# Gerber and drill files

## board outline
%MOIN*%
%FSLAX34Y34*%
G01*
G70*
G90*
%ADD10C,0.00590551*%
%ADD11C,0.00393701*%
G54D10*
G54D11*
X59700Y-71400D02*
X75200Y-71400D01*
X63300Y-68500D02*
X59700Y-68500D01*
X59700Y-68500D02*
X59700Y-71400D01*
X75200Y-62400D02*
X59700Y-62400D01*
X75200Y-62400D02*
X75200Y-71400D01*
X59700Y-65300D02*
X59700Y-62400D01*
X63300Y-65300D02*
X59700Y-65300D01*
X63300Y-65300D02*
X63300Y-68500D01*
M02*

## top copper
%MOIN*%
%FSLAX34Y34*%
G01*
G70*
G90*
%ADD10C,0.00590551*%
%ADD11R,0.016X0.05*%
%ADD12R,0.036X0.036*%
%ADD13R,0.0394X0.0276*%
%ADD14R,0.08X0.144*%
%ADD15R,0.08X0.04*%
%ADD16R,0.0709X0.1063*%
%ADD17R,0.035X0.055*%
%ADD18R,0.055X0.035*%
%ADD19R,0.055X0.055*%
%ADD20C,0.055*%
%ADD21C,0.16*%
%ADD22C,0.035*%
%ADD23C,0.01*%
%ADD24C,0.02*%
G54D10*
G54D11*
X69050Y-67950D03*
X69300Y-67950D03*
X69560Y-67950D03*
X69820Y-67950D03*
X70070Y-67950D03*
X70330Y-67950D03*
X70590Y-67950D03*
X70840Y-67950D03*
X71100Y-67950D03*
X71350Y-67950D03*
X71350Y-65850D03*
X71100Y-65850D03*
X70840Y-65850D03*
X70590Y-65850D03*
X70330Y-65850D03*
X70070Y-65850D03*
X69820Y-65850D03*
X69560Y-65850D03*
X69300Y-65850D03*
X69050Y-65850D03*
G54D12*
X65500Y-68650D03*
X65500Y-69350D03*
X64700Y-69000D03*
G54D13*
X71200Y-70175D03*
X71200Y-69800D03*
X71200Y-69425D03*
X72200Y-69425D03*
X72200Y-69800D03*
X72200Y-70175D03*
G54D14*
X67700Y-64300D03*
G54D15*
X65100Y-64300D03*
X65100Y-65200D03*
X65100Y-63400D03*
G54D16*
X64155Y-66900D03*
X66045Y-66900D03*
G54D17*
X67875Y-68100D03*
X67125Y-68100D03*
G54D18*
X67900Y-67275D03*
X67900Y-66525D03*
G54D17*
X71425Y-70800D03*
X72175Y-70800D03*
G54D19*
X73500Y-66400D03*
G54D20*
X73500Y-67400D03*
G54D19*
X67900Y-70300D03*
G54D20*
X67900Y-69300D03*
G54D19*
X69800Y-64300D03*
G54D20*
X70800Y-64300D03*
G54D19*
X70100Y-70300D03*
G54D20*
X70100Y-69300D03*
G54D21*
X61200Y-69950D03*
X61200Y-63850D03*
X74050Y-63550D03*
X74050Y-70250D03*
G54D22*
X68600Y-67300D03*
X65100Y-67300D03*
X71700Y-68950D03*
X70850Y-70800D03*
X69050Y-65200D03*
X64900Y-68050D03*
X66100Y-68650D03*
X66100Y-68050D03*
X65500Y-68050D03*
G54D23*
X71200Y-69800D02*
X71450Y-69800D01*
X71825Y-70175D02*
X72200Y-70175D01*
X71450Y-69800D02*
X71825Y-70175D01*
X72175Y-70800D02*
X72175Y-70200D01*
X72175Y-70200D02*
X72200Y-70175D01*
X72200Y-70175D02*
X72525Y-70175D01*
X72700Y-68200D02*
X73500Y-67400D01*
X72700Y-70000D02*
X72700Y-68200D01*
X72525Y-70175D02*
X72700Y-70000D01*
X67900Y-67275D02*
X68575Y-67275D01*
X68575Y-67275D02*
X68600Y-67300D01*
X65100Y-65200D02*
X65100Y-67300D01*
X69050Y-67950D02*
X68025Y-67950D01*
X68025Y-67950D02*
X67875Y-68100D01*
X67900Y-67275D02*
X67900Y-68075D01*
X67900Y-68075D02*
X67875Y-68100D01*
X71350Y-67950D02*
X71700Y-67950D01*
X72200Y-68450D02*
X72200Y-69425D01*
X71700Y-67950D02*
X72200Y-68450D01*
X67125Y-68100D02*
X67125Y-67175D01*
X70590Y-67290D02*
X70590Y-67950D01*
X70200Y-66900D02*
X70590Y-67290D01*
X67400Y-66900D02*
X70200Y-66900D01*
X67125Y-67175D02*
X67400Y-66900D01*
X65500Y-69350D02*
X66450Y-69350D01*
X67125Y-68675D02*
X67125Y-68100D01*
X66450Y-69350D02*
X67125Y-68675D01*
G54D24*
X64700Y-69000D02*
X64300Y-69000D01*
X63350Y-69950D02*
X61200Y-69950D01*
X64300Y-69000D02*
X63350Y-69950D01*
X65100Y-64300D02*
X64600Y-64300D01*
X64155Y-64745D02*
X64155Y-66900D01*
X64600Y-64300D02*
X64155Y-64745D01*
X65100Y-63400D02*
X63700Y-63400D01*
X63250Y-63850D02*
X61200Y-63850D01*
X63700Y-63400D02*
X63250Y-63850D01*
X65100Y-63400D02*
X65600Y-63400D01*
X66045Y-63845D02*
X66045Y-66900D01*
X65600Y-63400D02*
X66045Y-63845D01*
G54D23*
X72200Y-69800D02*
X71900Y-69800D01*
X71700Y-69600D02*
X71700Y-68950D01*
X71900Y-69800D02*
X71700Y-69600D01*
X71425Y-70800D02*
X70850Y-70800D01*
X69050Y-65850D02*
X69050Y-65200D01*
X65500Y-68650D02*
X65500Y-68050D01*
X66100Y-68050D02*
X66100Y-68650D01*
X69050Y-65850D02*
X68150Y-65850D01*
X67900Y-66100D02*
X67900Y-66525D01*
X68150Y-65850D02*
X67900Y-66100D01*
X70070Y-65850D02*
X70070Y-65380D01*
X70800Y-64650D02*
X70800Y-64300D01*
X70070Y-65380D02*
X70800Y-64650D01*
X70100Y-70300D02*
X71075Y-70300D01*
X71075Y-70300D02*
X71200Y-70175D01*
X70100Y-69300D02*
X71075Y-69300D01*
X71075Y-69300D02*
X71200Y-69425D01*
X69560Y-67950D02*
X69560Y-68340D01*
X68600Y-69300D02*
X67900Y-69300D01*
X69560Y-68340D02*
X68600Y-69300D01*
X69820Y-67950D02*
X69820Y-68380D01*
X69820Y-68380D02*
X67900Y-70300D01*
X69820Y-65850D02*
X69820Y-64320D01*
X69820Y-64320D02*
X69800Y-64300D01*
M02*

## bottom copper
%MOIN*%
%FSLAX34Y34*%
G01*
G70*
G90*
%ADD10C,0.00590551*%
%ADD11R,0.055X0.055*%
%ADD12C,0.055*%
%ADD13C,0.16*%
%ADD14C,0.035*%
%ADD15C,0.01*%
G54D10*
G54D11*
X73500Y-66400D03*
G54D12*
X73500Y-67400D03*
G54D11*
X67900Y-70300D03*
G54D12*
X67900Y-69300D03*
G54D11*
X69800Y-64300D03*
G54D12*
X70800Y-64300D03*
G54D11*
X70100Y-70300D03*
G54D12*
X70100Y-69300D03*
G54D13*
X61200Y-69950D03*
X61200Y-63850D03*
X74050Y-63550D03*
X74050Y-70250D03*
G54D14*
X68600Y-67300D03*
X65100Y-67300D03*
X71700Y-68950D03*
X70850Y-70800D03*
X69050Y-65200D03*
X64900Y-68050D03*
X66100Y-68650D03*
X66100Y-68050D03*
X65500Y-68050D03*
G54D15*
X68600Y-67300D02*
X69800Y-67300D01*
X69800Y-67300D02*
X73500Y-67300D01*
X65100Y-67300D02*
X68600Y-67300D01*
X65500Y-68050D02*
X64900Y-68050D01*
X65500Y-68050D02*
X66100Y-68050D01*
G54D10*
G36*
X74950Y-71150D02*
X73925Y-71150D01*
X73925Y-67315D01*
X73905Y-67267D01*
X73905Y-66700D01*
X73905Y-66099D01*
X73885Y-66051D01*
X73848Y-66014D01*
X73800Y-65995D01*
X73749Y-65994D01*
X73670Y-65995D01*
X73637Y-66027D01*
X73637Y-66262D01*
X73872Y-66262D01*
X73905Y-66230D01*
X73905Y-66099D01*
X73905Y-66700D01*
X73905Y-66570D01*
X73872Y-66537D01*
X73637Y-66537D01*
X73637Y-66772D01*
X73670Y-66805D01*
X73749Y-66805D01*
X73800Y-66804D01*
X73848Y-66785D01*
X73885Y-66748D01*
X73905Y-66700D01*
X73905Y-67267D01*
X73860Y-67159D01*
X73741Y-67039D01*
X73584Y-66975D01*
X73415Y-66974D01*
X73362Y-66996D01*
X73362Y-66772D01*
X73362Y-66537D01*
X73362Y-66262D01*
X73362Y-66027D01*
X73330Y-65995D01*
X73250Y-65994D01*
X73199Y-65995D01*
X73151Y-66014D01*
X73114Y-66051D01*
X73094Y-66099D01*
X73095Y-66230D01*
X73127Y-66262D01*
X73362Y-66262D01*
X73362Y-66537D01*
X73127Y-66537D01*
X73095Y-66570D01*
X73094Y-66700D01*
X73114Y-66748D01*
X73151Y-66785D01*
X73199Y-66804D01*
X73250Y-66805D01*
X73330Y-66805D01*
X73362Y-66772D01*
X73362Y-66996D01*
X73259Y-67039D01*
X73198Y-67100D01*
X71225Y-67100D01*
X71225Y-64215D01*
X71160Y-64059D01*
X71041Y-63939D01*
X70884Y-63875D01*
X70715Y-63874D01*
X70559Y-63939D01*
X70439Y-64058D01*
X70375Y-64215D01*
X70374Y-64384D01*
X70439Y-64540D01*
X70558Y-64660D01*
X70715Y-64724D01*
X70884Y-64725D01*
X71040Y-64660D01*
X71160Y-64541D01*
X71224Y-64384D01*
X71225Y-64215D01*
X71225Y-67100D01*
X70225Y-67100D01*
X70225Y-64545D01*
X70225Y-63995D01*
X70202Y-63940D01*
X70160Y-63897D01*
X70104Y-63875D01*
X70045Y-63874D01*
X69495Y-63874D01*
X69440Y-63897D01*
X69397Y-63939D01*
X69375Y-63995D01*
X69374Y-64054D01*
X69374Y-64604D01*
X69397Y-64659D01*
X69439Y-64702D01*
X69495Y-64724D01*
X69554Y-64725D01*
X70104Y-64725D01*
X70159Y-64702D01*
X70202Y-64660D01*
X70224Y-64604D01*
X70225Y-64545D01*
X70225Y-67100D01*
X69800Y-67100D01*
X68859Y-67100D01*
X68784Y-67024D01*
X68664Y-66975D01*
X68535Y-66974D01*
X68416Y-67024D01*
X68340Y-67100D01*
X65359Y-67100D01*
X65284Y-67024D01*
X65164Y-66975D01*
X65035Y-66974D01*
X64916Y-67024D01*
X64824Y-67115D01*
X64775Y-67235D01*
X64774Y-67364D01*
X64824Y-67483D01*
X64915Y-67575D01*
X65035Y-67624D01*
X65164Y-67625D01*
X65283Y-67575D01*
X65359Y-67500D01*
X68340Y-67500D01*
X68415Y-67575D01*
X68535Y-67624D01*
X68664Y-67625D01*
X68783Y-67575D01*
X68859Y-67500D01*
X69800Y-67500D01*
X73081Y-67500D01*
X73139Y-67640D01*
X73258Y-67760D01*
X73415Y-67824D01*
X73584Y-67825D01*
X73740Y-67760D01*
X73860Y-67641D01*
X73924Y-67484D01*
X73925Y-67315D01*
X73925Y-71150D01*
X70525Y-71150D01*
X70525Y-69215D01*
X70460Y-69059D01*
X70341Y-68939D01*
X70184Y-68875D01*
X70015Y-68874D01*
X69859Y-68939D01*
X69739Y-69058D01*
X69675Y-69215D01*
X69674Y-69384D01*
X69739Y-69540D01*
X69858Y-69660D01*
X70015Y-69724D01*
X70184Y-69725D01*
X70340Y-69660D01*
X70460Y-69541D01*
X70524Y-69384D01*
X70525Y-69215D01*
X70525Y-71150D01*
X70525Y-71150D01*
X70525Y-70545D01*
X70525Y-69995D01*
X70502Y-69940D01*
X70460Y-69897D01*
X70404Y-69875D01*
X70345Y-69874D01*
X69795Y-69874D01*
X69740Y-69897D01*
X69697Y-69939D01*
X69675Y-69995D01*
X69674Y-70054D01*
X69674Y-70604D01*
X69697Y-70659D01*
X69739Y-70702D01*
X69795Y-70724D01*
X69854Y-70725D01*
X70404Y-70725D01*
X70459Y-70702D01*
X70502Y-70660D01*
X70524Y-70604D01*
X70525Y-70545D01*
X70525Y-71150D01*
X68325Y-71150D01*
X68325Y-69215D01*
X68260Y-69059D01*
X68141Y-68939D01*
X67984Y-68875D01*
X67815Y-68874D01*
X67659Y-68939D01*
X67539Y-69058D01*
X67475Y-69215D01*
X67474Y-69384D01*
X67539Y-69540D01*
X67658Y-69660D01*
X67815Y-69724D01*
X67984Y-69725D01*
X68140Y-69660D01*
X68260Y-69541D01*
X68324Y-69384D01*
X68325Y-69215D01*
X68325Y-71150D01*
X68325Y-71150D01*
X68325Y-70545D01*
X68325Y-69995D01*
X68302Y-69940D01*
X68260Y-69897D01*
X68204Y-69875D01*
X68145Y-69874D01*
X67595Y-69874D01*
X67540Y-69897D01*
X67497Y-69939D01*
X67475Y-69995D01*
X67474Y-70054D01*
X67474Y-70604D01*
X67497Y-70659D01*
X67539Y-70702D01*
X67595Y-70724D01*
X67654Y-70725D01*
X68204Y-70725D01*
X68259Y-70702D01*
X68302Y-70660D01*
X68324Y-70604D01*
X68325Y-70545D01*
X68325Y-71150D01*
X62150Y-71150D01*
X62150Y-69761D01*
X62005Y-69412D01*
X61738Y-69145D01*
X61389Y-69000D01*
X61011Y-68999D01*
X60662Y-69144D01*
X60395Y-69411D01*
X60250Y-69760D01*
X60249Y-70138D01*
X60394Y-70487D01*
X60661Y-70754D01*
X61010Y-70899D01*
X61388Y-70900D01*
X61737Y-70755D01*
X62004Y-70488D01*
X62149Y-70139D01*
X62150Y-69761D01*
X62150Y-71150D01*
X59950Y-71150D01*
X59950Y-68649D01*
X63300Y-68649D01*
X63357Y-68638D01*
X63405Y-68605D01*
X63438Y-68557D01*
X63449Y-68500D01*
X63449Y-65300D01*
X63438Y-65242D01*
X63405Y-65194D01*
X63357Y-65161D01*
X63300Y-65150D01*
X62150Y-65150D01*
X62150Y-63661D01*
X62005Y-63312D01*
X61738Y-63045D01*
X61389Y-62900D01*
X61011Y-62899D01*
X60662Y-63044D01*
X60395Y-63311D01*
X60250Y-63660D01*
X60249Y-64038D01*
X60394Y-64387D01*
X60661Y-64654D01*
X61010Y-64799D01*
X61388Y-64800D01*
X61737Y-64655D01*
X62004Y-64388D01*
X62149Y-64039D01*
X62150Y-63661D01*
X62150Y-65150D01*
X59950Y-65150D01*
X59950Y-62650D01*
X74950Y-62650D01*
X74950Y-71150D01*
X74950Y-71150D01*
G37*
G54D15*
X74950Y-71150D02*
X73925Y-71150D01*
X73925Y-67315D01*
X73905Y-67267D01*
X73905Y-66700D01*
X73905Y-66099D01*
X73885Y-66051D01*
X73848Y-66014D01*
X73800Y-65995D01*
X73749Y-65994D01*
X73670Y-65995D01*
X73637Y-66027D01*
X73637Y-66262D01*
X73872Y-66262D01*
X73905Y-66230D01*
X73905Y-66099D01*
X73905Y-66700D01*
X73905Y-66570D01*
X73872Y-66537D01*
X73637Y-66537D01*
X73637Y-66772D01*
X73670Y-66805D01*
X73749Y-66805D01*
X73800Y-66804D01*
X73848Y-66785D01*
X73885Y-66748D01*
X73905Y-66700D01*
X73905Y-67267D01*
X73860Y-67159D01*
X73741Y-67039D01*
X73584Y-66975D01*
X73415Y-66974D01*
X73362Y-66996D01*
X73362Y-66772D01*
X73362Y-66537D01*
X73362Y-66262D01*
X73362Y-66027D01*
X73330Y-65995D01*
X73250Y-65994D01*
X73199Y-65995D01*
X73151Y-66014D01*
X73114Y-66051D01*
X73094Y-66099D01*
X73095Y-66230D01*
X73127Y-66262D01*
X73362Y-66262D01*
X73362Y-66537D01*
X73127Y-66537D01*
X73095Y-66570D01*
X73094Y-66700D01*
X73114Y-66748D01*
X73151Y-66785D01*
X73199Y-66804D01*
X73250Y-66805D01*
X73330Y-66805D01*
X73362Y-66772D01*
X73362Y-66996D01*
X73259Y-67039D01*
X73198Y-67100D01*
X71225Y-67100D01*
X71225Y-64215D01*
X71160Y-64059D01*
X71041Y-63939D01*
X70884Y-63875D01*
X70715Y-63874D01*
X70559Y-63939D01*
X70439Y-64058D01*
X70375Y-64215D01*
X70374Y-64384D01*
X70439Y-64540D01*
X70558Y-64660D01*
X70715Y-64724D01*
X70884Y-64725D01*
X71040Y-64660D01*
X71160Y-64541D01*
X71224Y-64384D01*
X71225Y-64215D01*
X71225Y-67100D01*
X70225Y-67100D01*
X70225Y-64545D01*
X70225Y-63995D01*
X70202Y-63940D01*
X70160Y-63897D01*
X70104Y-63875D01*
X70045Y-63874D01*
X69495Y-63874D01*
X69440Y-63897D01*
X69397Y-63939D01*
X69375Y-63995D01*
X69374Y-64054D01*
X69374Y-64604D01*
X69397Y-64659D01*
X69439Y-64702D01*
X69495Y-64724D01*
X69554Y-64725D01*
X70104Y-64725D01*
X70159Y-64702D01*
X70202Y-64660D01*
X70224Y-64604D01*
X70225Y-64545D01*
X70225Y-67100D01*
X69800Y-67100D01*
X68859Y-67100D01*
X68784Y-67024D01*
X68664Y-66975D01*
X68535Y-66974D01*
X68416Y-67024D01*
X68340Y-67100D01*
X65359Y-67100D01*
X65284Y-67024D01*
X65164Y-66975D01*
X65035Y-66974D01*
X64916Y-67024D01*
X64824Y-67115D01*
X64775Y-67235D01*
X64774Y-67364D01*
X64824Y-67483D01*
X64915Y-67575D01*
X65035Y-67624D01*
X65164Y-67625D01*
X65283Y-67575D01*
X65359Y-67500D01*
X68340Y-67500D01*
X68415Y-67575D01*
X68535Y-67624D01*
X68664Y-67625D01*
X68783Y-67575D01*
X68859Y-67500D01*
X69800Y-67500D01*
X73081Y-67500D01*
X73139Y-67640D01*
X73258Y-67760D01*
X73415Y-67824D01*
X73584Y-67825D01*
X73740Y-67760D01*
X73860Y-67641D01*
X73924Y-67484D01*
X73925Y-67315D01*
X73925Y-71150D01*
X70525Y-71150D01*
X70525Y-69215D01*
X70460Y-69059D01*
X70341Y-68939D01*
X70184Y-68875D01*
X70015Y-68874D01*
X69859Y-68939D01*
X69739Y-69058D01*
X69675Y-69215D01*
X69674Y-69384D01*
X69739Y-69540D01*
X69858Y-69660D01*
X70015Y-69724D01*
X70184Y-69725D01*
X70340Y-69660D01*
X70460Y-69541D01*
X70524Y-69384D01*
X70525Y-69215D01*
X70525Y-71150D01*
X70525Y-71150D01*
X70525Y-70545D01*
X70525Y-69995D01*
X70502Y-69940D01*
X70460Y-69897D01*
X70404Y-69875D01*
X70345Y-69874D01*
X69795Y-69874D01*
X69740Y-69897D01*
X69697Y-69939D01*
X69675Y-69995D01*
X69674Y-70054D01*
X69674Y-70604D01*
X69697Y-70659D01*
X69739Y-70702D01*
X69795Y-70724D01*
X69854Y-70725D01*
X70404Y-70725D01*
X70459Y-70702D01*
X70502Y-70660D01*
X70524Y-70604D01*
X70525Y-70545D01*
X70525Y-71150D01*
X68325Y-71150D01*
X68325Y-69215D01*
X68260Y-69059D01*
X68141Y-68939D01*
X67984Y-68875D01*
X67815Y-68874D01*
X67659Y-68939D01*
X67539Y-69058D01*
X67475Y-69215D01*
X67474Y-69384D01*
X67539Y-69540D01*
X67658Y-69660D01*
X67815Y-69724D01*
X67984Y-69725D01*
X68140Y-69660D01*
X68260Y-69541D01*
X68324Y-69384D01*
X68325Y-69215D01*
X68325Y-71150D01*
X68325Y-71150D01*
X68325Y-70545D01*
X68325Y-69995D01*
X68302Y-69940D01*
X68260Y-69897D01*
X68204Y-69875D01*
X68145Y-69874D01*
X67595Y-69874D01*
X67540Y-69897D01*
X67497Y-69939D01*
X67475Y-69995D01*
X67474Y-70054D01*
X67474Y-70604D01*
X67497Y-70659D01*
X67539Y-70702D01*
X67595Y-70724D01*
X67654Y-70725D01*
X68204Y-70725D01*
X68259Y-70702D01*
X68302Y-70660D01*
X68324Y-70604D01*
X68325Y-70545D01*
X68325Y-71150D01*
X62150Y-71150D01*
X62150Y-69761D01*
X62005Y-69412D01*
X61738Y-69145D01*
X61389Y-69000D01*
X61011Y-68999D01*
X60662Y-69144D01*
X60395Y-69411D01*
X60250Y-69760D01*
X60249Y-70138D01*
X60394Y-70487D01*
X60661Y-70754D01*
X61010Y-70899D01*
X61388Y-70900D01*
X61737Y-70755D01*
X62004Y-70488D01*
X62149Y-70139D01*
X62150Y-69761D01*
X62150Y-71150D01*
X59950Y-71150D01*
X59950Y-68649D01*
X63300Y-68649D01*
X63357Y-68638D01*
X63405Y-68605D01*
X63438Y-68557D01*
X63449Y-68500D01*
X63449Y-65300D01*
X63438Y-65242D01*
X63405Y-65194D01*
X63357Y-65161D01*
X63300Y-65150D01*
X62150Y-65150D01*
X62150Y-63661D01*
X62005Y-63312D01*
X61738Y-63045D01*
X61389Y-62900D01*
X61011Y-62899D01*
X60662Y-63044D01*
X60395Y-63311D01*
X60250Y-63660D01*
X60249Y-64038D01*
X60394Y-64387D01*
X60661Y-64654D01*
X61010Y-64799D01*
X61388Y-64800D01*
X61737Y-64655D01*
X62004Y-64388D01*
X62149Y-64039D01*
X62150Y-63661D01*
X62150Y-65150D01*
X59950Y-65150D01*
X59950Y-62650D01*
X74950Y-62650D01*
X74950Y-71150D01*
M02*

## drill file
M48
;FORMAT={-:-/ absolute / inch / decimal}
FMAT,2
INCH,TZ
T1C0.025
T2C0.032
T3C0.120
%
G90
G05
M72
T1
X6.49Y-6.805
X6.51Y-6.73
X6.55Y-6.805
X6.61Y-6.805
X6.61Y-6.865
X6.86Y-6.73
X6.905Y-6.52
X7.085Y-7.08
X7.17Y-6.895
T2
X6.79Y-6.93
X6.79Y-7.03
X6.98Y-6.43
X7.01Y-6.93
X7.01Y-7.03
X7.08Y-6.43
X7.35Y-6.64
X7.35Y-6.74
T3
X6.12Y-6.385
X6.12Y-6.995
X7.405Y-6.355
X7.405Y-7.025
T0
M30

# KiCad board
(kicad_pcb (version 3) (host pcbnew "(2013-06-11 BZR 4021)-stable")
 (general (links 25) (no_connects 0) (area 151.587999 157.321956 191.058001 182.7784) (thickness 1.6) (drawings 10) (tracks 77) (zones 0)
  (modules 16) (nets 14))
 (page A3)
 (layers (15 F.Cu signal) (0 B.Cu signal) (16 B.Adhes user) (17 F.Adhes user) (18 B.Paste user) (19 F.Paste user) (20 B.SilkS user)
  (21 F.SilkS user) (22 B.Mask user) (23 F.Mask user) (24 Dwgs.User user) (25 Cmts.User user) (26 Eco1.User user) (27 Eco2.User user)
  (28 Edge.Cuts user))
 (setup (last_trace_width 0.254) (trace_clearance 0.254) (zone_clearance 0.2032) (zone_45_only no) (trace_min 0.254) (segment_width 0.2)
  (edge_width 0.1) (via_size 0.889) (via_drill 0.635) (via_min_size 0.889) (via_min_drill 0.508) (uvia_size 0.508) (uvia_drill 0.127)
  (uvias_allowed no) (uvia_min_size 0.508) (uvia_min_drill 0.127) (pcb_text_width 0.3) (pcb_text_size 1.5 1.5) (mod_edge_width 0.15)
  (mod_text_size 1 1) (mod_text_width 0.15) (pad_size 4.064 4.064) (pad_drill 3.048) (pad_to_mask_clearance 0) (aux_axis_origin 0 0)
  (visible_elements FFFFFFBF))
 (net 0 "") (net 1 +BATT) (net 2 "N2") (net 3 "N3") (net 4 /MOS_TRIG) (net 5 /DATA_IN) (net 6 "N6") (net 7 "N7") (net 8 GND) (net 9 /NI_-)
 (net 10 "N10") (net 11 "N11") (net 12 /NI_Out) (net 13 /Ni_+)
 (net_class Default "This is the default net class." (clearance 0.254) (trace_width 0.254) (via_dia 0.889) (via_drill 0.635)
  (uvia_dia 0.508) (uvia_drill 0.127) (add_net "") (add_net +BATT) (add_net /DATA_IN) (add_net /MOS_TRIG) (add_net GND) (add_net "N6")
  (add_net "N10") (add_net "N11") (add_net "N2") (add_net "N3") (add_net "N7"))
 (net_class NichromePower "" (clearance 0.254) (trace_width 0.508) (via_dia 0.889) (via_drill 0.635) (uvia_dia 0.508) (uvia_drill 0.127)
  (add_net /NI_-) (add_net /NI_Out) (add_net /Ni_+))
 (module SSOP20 (layer F.Cu) (at 178.308 169.926)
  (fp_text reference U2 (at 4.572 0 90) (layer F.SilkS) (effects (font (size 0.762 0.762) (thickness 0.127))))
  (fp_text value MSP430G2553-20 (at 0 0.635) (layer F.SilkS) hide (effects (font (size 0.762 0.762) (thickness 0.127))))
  (pad 1 smd rect (at -2.921 2.667) (size 0.4064 1.27) (layers F.Cu F.Paste F.Mask) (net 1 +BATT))
  (pad 2 smd rect (at -2.286 2.667) (size 0.4064 1.27) (layers F.Cu F.Paste F.Mask))
  (pad 3 smd rect (at -1.6256 2.667) (size 0.4064 1.27) (layers F.Cu F.Paste F.Mask) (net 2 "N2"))
  (pad 4 smd rect (at -0.9652 2.667) (size 0.4064 1.27) (layers F.Cu F.Paste F.Mask) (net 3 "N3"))
  (pad 5 smd rect (at -0.3302 2.667) (size 0.4064 1.27) (layers F.Cu F.Paste F.Mask))
  (pad 6 smd rect (at 0.3302 2.667) (size 0.4064 1.27) (layers F.Cu F.Paste F.Mask))
  (pad 7 smd rect (at 0.9906 2.667) (size 0.4064 1.27) (layers F.Cu F.Paste F.Mask) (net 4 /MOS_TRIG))
  (pad 8 smd rect (at 1.6256 2.667) (size 0.4064 1.27) (layers F.Cu F.Paste F.Mask))
  (pad 9 smd rect (at 2.286 2.667) (size 0.4064 1.27) (layers F.Cu F.Paste F.Mask))
  (pad 10 smd rect (at 2.921 2.667) (size 0.4064 1.27) (layers F.Cu F.Paste F.Mask) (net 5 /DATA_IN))
  (pad 11 smd rect (at 2.921 -2.667) (size 0.4064 1.27) (layers F.Cu F.Paste F.Mask))
  (pad 12 smd rect (at 2.286 -2.667) (size 0.4064 1.27) (layers F.Cu F.Paste F.Mask))
  (pad 13 smd rect (at 1.6256 -2.667) (size 0.4064 1.27) (layers F.Cu F.Paste F.Mask))
  (pad 14 smd rect (at 0.9906 -2.667) (size 0.4064 1.27) (layers F.Cu F.Paste F.Mask))
  (pad 15 smd rect (at 0.3302 -2.667) (size 0.4064 1.27) (layers F.Cu F.Paste F.Mask))
  (pad 16 smd rect (at -0.3302 -2.667) (size 0.4064 1.27) (layers F.Cu F.Paste F.Mask) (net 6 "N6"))
  (pad 17 smd rect (at -0.9652 -2.667) (size 0.4064 1.27) (layers F.Cu F.Paste F.Mask) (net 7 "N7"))
  (pad 18 smd rect (at -1.6256 -2.667) (size 0.4064 1.27) (layers F.Cu F.Paste F.Mask))
  (pad 19 smd rect (at -2.286 -2.667) (size 0.4064 1.27) (layers F.Cu F.Paste F.Mask))
  (pad 20 smd rect (at -2.921 -2.667) (size 0.4064 1.27) (layers F.Cu F.Paste F.Mask) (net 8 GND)))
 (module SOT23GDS (layer F.Cu) (at 165.354 175.26 270)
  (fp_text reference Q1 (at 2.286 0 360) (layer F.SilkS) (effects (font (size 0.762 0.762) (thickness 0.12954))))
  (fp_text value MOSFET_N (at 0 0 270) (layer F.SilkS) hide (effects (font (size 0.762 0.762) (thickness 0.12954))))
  (pad S smd rect (at -0.889 -1.016 270) (size 0.9144 0.9144) (layers F.Cu F.Paste F.Mask) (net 8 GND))
  (pad G smd rect (at 0.889 -1.016 270) (size 0.9144 0.9144) (layers F.Cu F.Paste F.Mask) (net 4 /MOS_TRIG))
  (pad D smd rect (at 0 1.016 270) (size 0.9144 0.9144) (layers F.Cu F.Paste F.Mask) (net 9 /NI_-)))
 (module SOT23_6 (layer F.Cu) (at 182.118 177.292 90)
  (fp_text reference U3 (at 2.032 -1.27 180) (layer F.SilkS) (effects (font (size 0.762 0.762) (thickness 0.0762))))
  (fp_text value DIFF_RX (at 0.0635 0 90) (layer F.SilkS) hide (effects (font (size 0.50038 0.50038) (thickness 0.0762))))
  (pad 6 smd rect (at -0.9525 -1.27 90) (size 0.70104 1.00076) (layers F.Cu F.Paste F.Mask) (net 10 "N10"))
  (pad 5 smd rect (at 0 -1.27 90) (size 0.70104 1.00076) (layers F.Cu F.Paste F.Mask) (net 1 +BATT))
  (pad 4 smd rect (at 0.9525 -1.27 90) (size 0.70104 1.00076) (layers F.Cu F.Paste F.Mask) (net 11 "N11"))
  (pad 3 smd rect (at 0.9525 1.27 90) (size 0.70104 1.00076) (layers F.Cu F.Paste F.Mask) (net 5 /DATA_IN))
  (pad 2 smd rect (at 0 1.27 90) (size 0.70104 1.00076) (layers F.Cu F.Paste F.Mask) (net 8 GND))
  (pad 1 smd rect (at -0.9525 1.27 90) (size 0.70104 1.00076) (layers F.Cu F.Paste F.Mask) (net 1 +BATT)))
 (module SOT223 (layer F.Cu) (at 168.656 163.322 270)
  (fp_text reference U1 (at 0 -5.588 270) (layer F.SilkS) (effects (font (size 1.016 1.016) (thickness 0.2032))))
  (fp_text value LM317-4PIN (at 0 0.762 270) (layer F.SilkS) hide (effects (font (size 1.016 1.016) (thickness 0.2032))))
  (pad 4 smd rect (at 0 -3.302 270) (size 3.6576 2.032) (layers F.Cu F.Paste F.Mask))
  (pad 2 smd rect (at 0 3.302 270) (size 1.016 2.032) (layers F.Cu F.Paste F.Mask) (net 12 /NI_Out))
  (pad 3 smd rect (at 2.286 3.302 270) (size 1.016 2.032) (layers F.Cu F.Paste F.Mask) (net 1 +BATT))
  (pad 1 smd rect (at -2.286 3.302 270) (size 1.016 2.032) (layers F.Cu F.Paste F.Mask) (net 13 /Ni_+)))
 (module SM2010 (layer F.Cu) (at 165.354 169.926)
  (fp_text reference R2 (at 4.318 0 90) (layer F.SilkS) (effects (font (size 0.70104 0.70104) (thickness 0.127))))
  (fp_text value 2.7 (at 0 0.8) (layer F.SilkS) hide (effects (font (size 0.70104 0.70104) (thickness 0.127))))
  (pad 1 smd rect (at -2.4003 0) (size 1.80086 2.70002) (layers F.Cu F.Paste F.Mask) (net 12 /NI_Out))
  (pad 2 smd rect (at 2.4003 0) (size 1.80086 2.70002) (layers F.Cu F.Paste F.Mask) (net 13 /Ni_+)))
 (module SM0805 (layer F.Cu) (at 171.45 172.974 180)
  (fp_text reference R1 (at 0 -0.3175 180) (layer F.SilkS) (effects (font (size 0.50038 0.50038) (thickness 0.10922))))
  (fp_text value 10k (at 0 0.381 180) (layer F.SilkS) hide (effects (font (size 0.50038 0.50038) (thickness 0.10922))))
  (pad 1 smd rect (at -0.9525 0 180) (size 0.889 1.397) (layers F.Cu F.Paste F.Mask) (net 1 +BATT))
  (pad 2 smd rect (at 0.9525 0 180) (size 0.889 1.397) (layers F.Cu F.Paste F.Mask) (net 4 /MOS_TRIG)))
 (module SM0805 (layer F.Cu) (at 172.466 169.926 90)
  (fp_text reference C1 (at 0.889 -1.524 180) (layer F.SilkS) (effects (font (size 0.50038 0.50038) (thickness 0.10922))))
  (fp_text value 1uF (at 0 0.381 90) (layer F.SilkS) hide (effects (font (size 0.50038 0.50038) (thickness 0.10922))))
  (pad 1 smd rect (at -0.9525 0 90) (size 0.889 1.397) (layers F.Cu F.Paste F.Mask) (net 1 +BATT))
  (pad 2 smd rect (at 0.9525 0 90) (size 0.889 1.397) (layers F.Cu F.Paste F.Mask) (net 8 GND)))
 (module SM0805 (layer F.Cu) (at 182.372 179.832)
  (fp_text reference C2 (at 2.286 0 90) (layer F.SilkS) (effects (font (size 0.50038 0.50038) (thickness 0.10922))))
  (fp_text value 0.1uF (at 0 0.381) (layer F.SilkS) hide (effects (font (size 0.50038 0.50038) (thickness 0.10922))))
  (pad 1 smd rect (at -0.9525 0) (size 0.889 1.397) (layers F.Cu F.Paste F.Mask) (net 8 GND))
  (pad 2 smd rect (at 0.9525 0) (size 0.889 1.397) (layers F.Cu F.Paste F.Mask) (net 1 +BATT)))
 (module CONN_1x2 (layer F.Cu) (at 186.69 169.926 90)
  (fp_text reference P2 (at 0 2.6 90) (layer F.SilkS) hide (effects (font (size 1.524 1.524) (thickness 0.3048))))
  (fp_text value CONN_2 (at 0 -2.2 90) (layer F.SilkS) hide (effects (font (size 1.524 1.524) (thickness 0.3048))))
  (pad 1 thru_hole rect (at 1.27 0 90) (size 1.397 1.397) (drill 0.8128) (layers *.Cu *.Mask F.SilkS) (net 8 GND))
  (pad 2 thru_hole circle (at -1.27 0 90) (size 1.397 1.397) (drill 0.8128) (layers *.Cu *.Mask F.SilkS) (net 1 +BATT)))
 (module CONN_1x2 (layer F.Cu) (at 172.466 177.292 270)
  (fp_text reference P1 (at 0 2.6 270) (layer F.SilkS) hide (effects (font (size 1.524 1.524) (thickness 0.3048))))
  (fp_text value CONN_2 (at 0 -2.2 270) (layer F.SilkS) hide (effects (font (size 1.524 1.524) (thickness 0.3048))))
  (pad 1 thru_hole rect (at 1.27 0 270) (size 1.397 1.397) (drill 0.8128) (layers *.Cu *.Mask F.SilkS) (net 3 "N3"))
  (pad 2 thru_hole circle (at -1.27 0 270) (size 1.397 1.397) (drill 0.8128) (layers *.Cu *.Mask F.SilkS) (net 2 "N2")))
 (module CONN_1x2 (layer F.Cu) (at 178.562 163.322 180)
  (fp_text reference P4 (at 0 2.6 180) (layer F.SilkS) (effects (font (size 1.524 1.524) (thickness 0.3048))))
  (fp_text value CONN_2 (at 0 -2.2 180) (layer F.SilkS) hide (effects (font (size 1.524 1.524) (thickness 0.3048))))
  (pad 1 thru_hole rect (at 1.27 0 180) (size 1.397 1.397) (drill 0.8128) (layers *.Cu *.Mask F.SilkS) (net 7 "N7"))
  (pad 2 thru_hole circle (at -1.27 0 180) (size 1.397 1.397) (drill 0.8128) (layers *.Cu *.Mask F.SilkS) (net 6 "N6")))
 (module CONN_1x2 (layer F.Cu) (at 178.054 177.292 270)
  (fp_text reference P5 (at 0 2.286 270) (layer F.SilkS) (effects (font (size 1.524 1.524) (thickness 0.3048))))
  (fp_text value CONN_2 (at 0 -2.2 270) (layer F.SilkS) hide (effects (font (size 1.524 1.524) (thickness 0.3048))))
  (pad 1 thru_hole rect (at 1.27 0 270) (size 1.397 1.397) (drill 0.8128) (layers *.Cu *.Mask F.SilkS) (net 10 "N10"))
  (pad 2 thru_hole circle (at -1.27 0 270) (size 1.397 1.397) (drill 0.8128) (layers *.Cu *.Mask F.SilkS) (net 11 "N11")))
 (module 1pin (layer F.Cu) (at 155.448 177.673)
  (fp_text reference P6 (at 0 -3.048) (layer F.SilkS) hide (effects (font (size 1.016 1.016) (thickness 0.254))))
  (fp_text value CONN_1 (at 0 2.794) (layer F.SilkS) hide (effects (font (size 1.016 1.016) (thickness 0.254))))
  (pad 1 thru_hole circle (at 0 0) (size 4.064 4.064) (drill 3.048) (layers *.Cu *.Mask F.SilkS) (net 9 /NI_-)))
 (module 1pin (layer F.Cu) (at 155.448 162.179)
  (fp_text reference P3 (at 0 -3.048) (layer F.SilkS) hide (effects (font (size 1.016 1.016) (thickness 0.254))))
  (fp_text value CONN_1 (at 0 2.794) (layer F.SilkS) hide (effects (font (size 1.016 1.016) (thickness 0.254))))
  (pad 1 thru_hole circle (at 0 0) (size 4.064 4.064) (drill 3.048) (layers *.Cu *.Mask F.SilkS) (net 13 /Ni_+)))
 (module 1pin (layer F.Cu) (at 188.087 161.417)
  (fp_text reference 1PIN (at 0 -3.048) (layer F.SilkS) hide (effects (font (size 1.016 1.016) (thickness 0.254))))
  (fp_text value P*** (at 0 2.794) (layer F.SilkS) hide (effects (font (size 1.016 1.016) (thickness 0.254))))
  (pad 1 thru_hole circle (at 0 0) (size 4.064 4.064) (drill 3.048) (layers *.Cu *.Mask F.SilkS)))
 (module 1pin (layer F.Cu) (at 188.087 178.435)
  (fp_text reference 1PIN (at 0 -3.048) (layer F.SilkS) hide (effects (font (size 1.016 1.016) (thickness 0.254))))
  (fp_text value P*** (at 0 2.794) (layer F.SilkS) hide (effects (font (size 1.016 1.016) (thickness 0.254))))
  (pad 1 thru_hole circle (at 0 0) (size 4.064 4.064) (drill 3.048) (layers *.Cu *.Mask F.SilkS)))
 (gr_line (start 151.638 181.356) (end 191.008 181.356) (angle 90) (layer Edge.Cuts) (width 0.1))
 (gr_line (start 160.782 173.99) (end 151.638 173.99) (angle 90) (layer Edge.Cuts) (width 0.1))
 (gr_line (start 151.638 173.99) (end 151.638 181.356) (angle 90) (layer Edge.Cuts) (width 0.1))
 (gr_line (start 191.008 158.496) (end 151.638 158.496) (angle 90) (layer Edge.Cuts) (width 0.1))
 (gr_line (start 191.008 158.496) (end 191.008 181.356) (angle 90) (layer Edge.Cuts) (width 0.1))
 (gr_line (start 151.638 165.862) (end 151.638 158.496) (angle 90) (layer Edge.Cuts) (width 0.1))
 (gr_line (start 160.782 165.862) (end 151.638 165.862) (angle 90) (layer Edge.Cuts) (width 0.1))
 (gr_line (start 160.782 165.862) (end 160.782 173.99) (angle 90) (layer Edge.Cuts) (width 0.1))
 (segment (start 180.848 177.292) (end 181.483 177.292) (width 0.254) (layer F.Cu) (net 1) (status 400000))
 (segment (start 182.4355 178.2445) (end 183.388 178.2445) (width 0.254) (layer F.Cu) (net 1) (status 800000))
 (segment (start 181.483 177.292) (end 182.4355 178.2445) (width 0.254) (layer F.Cu) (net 1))
 (segment (start 183.3245 179.832) (end 183.3245 178.308) (width 0.254) (layer F.Cu) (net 1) (status C00000))
 (segment (start 183.3245 178.308) (end 183.388 178.2445) (width 0.254) (layer F.Cu) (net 1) (status C00000))
 (segment (start 183.388 178.2445) (end 184.2135 178.2445) (width 0.254) (layer F.Cu) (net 1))
 (segment (start 184.658 173.228) (end 186.69 171.196) (width 0.254) (layer F.Cu) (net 1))
 (segment (start 184.658 177.8) (end 184.658 173.228) (width 0.254) (layer F.Cu) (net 1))
 (segment (start 184.2135 178.2445) (end 184.658 177.8) (width 0.254) (layer F.Cu) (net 1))
 (segment (start 172.466 170.8785) (end 174.1805 170.8785) (width 0.254) (layer F.Cu) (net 1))
 (via (at 174.244 170.942) (size 0.889) (layers F.Cu B.Cu) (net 1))
 (segment (start 174.1805 170.8785) (end 174.244 170.942) (width 0.254) (layer F.Cu) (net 1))
 (segment (start 174.244 170.942) (end 177.292 170.942) (width 0.254) (layer B.Cu) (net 1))
 (segment (start 177.292 170.942) (end 186.69 170.942) (width 0.254) (layer B.Cu) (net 1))
 (segment (start 165.354 165.608) (end 165.354 170.942) (width 0.254) (layer F.Cu) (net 1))
 (via (at 165.354 170.942) (size 0.889) (layers F.Cu B.Cu) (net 1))
 (segment (start 165.354 170.942) (end 174.244 170.942) (width 0.254) (layer B.Cu) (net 1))
 (segment (start 175.387 172.593) (end 172.7835 172.593) (width 0.254) (layer F.Cu) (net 1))
 (segment (start 172.7835 172.593) (end 172.4025 172.974) (width 0.254) (layer F.Cu) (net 1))
 (segment (start 172.466 170.8785) (end 172.466 172.9105) (width 0.254) (layer F.Cu) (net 1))
 (segment (start 172.466 172.9105) (end 172.4025 172.974) (width 0.254) (layer F.Cu) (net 1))
 (segment (start 181.229 172.593) (end 182.118 172.593) (width 0.254) (layer F.Cu) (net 5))
 (segment (start 183.388 173.863) (end 183.388 176.3395) (width 0.254) (layer F.Cu) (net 5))
 (segment (start 182.118 172.593) (end 183.388 173.863) (width 0.254) (layer F.Cu) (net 5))
 (segment (start 170.4975 172.974) (end 170.4975 170.6245) (width 0.254) (layer F.Cu) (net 4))
 (segment (start 179.2986 170.9166) (end 179.2986 172.593) (width 0.254) (layer F.Cu) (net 4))
 (segment (start 178.308 169.926) (end 179.2986 170.9166) (width 0.254) (layer F.Cu) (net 4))
 (segment (start 171.196 169.926) (end 178.308 169.926) (width 0.254) (layer F.Cu) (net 4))
 (segment (start 170.4975 170.6245) (end 171.196 169.926) (width 0.254) (layer F.Cu) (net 4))
 (segment (start 166.37 176.149) (end 168.783 176.149) (width 0.254) (layer F.Cu) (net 4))
 (segment (start 170.4975 174.4345) (end 170.4975 172.974) (width 0.254) (layer F.Cu) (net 4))
 (segment (start 168.783 176.149) (end 170.4975 174.4345) (width 0.254) (layer F.Cu) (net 4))
 (segment (start 164.338 175.26) (end 163.322 175.26) (width 0.508) (layer F.Cu) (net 9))
 (segment (start 160.909 177.673) (end 155.448 177.673) (width 0.508) (layer F.Cu) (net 9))
 (segment (start 163.322 175.26) (end 160.909 177.673) (width 0.508) (layer F.Cu) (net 9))
 (segment (start 165.354 163.322) (end 164.084 163.322) (width 0.508) (layer F.Cu) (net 12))
 (segment (start 162.9537 164.4523) (end 162.9537 169.926) (width 0.508) (layer F.Cu) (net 12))
 (segment (start 164.084 163.322) (end 162.9537 164.4523) (width 0.508) (layer F.Cu) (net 12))
 (segment (start 165.354 161.036) (end 161.798 161.036) (width 0.508) (layer F.Cu) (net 13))
 (segment (start 160.655 162.179) (end 155.448 162.179) (width 0.508) (layer F.Cu) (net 13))
 (segment (start 161.798 161.036) (end 160.655 162.179) (width 0.508) (layer F.Cu) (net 13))
 (segment (start 165.354 161.036) (end 166.624 161.036) (width 0.508) (layer F.Cu) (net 13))
 (segment (start 167.7543 162.1663) (end 167.7543 169.926) (width 0.508) (layer F.Cu) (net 13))
 (segment (start 166.624 161.036) (end 167.7543 162.1663) (width 0.508) (layer F.Cu) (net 13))
 (segment (start 183.388 177.292) (end 182.626 177.292) (width 0.254) (layer F.Cu) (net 8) (status 400000))
 (via (at 182.118 175.133) (size 0.889) (layers F.Cu B.Cu) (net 8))
 (segment (start 182.118 176.784) (end 182.118 175.133) (width 0.254) (layer F.Cu) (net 8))
 (segment (start 182.626 177.292) (end 182.118 176.784) (width 0.254) (layer F.Cu) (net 8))
 (via (at 179.959 179.832) (size 0.889) (layers F.Cu B.Cu) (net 8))
 (segment (start 181.4195 179.832) (end 179.959 179.832) (width 0.254) (layer F.Cu) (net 8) (status 400000))
 (via (at 175.387 165.608) (size 0.889) (layers F.Cu B.Cu) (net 8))
 (segment (start 175.387 167.259) (end 175.387 165.608) (width 0.254) (layer F.Cu) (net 8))
 (segment (start 166.37 172.847) (end 164.846 172.847) (width 0.254) (layer B.Cu) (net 8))
 (via (at 164.846 172.847) (size 0.889) (layers F.Cu B.Cu) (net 8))
 (segment (start 166.37 174.371) (end 166.37 172.847) (width 0.254) (layer F.Cu) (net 8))
 (via (at 167.894 174.371) (size 0.889) (layers F.Cu B.Cu) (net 8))
 (segment (start 167.894 172.847) (end 167.894 174.371) (width 0.254) (layer F.Cu) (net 8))
 (via (at 167.894 172.847) (size 0.889) (layers F.Cu B.Cu) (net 8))
 (segment (start 166.37 172.847) (end 167.894 172.847) (width 0.254) (layer B.Cu) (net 8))
 (via (at 166.37 172.847) (size 0.889) (layers F.Cu B.Cu) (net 8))
 (segment (start 175.387 167.259) (end 173.101 167.259) (width 0.254) (layer F.Cu) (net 8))
 (segment (start 172.466 167.894) (end 172.466 168.9735) (width 0.254) (layer F.Cu) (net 8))
 (segment (start 173.101 167.259) (end 172.466 167.894) (width 0.254) (layer F.Cu) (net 8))
 (segment (start 177.9778 167.259) (end 177.9778 166.0652) (width 0.254) (layer F.Cu) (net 6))
 (segment (start 179.832 164.211) (end 179.832 163.322) (width 0.254) (layer F.Cu) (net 6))
 (segment (start 177.9778 166.0652) (end 179.832 164.211) (width 0.254) (layer F.Cu) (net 6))
 (segment (start 178.054 178.562) (end 180.5305 178.562) (width 0.254) (layer F.Cu) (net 10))
 (segment (start 180.5305 178.562) (end 180.848 178.2445) (width 0.254) (layer F.Cu) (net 10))
 (segment (start 178.054 176.022) (end 180.5305 176.022) (width 0.254) (layer F.Cu) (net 11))
 (segment (start 180.5305 176.022) (end 180.848 176.3395) (width 0.254) (layer F.Cu) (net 11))
 (segment (start 176.6824 172.593) (end 176.6824 173.5836) (width 0.254) (layer F.Cu) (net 2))
 (segment (start 174.244 176.022) (end 172.466 176.022) (width 0.254) (layer F.Cu) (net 2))
 (segment (start 176.6824 173.5836) (end 174.244 176.022) (width 0.254) (layer F.Cu) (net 2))
 (segment (start 177.3428 172.593) (end 177.3428 173.6852) (width 0.254) (layer F.Cu) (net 3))
 (segment (start 177.3428 173.6852) (end 172.466 178.562) (width 0.254) (layer F.Cu) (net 3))
 (segment (start 177.3428 167.259) (end 177.3428 163.3728) (width 0.254) (layer F.Cu) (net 7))
 (segment (start 177.3428 163.3728) (end 177.292 163.322) (width 0.254) (layer F.Cu) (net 7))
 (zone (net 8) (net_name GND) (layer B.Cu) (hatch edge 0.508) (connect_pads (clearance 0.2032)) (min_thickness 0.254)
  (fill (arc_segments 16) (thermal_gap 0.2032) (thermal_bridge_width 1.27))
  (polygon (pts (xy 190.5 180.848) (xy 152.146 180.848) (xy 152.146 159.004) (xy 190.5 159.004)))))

